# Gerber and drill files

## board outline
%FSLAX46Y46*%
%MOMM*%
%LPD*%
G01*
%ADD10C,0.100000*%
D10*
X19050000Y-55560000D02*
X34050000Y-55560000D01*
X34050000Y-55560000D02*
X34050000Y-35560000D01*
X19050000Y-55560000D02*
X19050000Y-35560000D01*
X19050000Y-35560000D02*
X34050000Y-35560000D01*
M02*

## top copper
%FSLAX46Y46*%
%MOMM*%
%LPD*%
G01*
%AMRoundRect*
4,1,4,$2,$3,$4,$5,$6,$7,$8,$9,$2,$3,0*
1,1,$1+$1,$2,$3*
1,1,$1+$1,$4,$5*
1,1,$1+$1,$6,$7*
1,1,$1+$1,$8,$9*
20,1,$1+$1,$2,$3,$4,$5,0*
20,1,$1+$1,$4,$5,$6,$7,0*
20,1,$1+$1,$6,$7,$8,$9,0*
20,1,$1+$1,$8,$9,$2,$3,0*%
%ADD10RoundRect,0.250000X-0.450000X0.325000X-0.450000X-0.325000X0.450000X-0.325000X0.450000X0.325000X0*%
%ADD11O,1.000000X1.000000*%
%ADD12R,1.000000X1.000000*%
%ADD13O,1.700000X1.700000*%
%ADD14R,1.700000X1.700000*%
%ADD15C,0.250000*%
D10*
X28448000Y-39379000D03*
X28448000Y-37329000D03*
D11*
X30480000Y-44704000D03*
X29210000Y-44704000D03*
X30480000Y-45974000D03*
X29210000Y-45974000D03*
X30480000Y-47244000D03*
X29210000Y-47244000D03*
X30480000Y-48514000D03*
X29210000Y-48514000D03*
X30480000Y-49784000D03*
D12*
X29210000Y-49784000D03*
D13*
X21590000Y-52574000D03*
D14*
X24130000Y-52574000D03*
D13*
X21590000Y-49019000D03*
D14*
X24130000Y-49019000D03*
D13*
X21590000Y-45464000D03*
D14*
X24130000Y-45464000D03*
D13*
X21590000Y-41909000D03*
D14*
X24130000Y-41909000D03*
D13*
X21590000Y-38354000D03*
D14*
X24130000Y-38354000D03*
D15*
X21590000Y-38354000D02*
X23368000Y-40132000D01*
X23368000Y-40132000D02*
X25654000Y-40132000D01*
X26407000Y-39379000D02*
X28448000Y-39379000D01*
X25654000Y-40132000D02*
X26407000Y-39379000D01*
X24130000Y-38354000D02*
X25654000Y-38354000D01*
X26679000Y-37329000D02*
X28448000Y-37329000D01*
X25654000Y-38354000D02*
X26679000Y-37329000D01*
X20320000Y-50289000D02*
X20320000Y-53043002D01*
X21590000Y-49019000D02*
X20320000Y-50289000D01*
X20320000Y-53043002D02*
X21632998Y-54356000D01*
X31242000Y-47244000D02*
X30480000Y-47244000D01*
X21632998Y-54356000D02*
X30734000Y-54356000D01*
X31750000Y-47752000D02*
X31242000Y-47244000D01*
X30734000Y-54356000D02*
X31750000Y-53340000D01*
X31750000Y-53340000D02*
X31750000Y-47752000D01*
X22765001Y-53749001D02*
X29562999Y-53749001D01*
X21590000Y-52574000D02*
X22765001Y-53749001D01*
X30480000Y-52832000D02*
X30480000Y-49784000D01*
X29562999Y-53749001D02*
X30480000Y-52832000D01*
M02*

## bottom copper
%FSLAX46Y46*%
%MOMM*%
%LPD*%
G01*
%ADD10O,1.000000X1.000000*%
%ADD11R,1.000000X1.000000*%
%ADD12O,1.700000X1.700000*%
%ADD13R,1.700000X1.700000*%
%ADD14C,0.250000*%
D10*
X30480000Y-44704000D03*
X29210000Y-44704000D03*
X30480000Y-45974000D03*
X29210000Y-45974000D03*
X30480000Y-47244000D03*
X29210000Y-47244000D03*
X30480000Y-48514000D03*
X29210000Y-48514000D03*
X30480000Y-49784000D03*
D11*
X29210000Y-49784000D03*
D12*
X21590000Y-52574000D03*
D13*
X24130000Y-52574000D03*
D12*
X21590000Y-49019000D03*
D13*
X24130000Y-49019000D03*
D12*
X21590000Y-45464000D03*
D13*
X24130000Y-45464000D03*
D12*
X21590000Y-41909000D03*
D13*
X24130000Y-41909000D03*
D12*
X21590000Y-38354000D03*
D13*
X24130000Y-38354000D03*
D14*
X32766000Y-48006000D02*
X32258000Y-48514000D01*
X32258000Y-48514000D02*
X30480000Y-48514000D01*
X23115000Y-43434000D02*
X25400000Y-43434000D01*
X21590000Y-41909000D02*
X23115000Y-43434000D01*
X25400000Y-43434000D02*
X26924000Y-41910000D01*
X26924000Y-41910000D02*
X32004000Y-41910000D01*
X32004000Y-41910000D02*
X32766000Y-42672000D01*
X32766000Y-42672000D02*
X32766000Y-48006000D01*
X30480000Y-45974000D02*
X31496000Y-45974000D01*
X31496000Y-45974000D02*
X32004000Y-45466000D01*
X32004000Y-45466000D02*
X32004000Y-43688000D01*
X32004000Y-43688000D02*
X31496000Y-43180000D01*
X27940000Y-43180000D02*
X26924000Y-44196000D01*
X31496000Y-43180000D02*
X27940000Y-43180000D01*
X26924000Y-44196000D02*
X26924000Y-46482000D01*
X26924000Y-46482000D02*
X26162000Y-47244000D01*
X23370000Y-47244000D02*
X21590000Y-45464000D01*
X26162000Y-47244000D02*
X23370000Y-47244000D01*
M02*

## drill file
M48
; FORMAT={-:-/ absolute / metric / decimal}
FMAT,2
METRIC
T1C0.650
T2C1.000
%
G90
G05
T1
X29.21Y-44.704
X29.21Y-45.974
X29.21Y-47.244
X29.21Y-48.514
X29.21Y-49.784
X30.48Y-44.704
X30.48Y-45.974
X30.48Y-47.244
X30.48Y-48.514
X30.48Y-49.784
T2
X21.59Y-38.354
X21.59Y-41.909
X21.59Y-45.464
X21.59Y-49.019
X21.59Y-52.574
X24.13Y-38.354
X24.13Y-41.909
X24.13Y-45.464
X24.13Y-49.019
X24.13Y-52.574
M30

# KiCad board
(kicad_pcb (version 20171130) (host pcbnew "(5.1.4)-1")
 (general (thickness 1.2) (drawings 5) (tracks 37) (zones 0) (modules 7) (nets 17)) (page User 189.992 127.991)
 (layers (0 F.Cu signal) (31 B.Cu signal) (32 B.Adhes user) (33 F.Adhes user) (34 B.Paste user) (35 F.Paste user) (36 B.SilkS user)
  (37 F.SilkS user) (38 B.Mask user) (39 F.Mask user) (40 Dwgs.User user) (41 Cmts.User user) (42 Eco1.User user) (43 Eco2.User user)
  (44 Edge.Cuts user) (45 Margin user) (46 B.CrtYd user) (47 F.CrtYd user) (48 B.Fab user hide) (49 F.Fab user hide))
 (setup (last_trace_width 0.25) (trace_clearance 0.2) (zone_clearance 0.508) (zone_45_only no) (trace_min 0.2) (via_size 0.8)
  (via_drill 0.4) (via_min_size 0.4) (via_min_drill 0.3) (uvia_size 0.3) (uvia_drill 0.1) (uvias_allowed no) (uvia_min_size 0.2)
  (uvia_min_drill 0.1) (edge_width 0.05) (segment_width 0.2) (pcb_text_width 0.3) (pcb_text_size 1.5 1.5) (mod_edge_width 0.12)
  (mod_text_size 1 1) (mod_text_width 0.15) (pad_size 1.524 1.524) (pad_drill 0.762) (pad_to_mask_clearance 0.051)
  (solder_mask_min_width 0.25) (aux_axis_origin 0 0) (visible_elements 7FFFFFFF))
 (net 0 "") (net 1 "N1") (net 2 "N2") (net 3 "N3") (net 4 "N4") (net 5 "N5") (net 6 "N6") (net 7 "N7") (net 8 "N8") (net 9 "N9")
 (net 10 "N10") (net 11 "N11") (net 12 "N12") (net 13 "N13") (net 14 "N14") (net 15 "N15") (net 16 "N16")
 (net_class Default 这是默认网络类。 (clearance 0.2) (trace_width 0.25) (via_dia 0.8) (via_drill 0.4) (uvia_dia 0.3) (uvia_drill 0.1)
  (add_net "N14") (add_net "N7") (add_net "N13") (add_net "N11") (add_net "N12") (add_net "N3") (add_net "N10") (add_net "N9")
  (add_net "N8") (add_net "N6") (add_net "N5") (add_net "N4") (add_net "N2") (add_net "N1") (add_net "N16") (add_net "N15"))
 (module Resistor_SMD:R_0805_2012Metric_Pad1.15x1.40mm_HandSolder (layer F.Cu) (at 28.448 38.354 270)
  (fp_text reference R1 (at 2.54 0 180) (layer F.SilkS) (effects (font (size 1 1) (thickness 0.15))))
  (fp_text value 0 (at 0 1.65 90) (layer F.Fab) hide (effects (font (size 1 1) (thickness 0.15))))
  (pad 2 smd roundrect (at 1.025 0 270) (size 1.15 1.4) (layers F.Cu F.Paste F.Mask) (roundrect_rratio 0.217391) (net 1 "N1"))
  (pad 1 smd roundrect (at -1.025 0 270) (size 1.15 1.4) (layers F.Cu F.Paste F.Mask) (roundrect_rratio 0.217391) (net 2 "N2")))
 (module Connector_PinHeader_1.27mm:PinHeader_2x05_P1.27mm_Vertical (layer B.Cu) (at 29.21 49.784)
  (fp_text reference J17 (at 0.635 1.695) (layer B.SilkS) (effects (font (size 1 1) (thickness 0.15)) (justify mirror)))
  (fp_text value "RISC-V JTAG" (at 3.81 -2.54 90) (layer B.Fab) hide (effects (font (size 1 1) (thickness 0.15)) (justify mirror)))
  (pad 10 thru_hole oval (at 1.27 -5.08) (size 1 1) (drill 0.65) (layers *.Cu *.Mask) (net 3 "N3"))
  (pad 9 thru_hole oval (at 0 -5.08) (size 1 1) (drill 0.65) (layers *.Cu *.Mask) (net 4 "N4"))
  (pad 8 thru_hole oval (at 1.27 -3.81) (size 1 1) (drill 0.65) (layers *.Cu *.Mask) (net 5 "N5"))
  (pad 7 thru_hole oval (at 0 -3.81) (size 1 1) (drill 0.65) (layers *.Cu *.Mask) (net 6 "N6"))
  (pad 6 thru_hole oval (at 1.27 -2.54) (size 1 1) (drill 0.65) (layers *.Cu *.Mask) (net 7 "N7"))
  (pad 5 thru_hole oval (at 0 -2.54) (size 1 1) (drill 0.65) (layers *.Cu *.Mask) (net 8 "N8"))
  (pad 4 thru_hole oval (at 1.27 -1.27) (size 1 1) (drill 0.65) (layers *.Cu *.Mask) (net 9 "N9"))
  (pad 3 thru_hole oval (at 0 -1.27) (size 1 1) (drill 0.65) (layers *.Cu *.Mask) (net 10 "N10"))
  (pad 2 thru_hole oval (at 1.27 0) (size 1 1) (drill 0.65) (layers *.Cu *.Mask) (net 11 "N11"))
  (pad 1 thru_hole rect (at 0 0) (size 1 1) (drill 0.65) (layers *.Cu *.Mask) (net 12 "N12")))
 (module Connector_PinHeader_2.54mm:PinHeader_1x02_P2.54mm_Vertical (layer F.Cu) (at 24.13 52.574 270)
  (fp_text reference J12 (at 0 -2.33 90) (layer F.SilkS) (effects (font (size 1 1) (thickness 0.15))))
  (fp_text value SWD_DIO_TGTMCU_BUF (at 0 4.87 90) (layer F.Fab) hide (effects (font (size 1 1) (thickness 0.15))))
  (pad 2 thru_hole oval (at 0 2.54 270) (size 1.7 1.7) (drill 1) (layers *.Cu *.Mask) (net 11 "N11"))
  (pad 1 thru_hole rect (at 0 0 270) (size 1.7 1.7) (drill 1) (layers *.Cu *.Mask) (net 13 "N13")))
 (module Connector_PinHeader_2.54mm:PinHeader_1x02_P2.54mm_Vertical (layer F.Cu) (at 24.13 49.019 270)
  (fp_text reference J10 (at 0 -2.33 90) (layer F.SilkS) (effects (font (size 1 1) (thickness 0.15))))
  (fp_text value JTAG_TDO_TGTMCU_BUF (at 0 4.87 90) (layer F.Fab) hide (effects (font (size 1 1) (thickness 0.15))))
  (pad 2 thru_hole oval (at 0 2.54 270) (size 1.7 1.7) (drill 1) (layers *.Cu *.Mask) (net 7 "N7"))
  (pad 1 thru_hole rect (at 0 0 270) (size 1.7 1.7) (drill 1) (layers *.Cu *.Mask) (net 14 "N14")))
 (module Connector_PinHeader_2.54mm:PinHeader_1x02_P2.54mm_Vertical (layer F.Cu) (at 24.13 45.464 270)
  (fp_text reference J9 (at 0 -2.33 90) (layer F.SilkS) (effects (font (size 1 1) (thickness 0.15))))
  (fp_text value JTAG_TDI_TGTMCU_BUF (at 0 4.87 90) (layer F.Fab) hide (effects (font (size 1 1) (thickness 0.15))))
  (pad 2 thru_hole oval (at 0 2.54 270) (size 1.7 1.7) (drill 1) (layers *.Cu *.Mask) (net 5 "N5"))
  (pad 1 thru_hole rect (at 0 0 270) (size 1.7 1.7) (drill 1) (layers *.Cu *.Mask) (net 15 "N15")))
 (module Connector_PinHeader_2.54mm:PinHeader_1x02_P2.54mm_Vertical (layer F.Cu) (at 24.13 41.909 270)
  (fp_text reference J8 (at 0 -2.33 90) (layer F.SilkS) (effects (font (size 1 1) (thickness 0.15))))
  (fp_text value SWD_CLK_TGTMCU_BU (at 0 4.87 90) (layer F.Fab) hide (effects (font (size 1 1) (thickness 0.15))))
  (pad 2 thru_hole oval (at 0 2.54 270) (size 1.7 1.7) (drill 1) (layers *.Cu *.Mask) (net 9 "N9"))
  (pad 1 thru_hole rect (at 0 0 270) (size 1.7 1.7) (drill 1) (layers *.Cu *.Mask) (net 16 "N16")))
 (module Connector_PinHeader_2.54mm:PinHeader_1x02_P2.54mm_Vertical (layer F.Cu) (at 24.13 38.354 270)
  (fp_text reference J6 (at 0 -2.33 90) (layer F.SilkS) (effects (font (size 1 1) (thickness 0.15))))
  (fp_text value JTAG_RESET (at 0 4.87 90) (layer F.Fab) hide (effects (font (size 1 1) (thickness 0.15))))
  (pad 2 thru_hole oval (at 0 2.54 270) (size 1.7 1.7) (drill 1) (layers *.Cu *.Mask) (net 1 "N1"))
  (pad 1 thru_hole rect (at 0 0 270) (size 1.7 1.7) (drill 1) (layers *.Cu *.Mask) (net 2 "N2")))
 (gr_line (start 19.05 55.56) (end 34.05 55.56) (layer Edge.Cuts) (width 0.1))
 (gr_line (start 34.05 55.56) (end 34.05 35.56) (layer Edge.Cuts) (width 0.1))
 (gr_line (start 19.05 55.56) (end 19.05 35.56) (layer Edge.Cuts) (width 0.1))
 (gr_line (start 19.05 35.56) (end 34.05 35.56) (layer Edge.Cuts) (width 0.1))
 (segment (start 21.59 38.354) (end 23.368 40.132) (width 0.25) (layer F.Cu) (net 1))
 (segment (start 23.368 40.132) (end 25.654 40.132) (width 0.25) (layer F.Cu) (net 1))
 (segment (start 26.407 39.379) (end 28.448 39.379) (width 0.25) (layer F.Cu) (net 1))
 (segment (start 25.654 40.132) (end 26.407 39.379) (width 0.25) (layer F.Cu) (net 1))
 (segment (start 24.13 38.354) (end 25.654 38.354) (width 0.25) (layer F.Cu) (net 2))
 (segment (start 26.679 37.329) (end 28.448 37.329) (width 0.25) (layer F.Cu) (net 2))
 (segment (start 25.654 38.354) (end 26.679 37.329) (width 0.25) (layer F.Cu) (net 2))
 (segment (start 32.766 48.006) (end 32.258 48.514) (width 0.25) (layer B.Cu) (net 9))
 (segment (start 32.258 48.514) (end 30.48 48.514) (width 0.25) (layer B.Cu) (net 9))
 (segment (start 23.115 43.434) (end 25.4 43.434) (width 0.25) (layer B.Cu) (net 9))
 (segment (start 21.59 41.909) (end 23.115 43.434) (width 0.25) (layer B.Cu) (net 9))
 (segment (start 25.4 43.434) (end 26.924 41.91) (width 0.25) (layer B.Cu) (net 9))
 (segment (start 26.924 41.91) (end 32.004 41.91) (width 0.25) (layer B.Cu) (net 9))
 (segment (start 32.004 41.91) (end 32.766 42.672) (width 0.25) (layer B.Cu) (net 9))
 (segment (start 32.766 42.672) (end 32.766 48.006) (width 0.25) (layer B.Cu) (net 9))
 (segment (start 30.48 45.974) (end 31.496 45.974) (width 0.25) (layer B.Cu) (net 5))
 (segment (start 31.496 45.974) (end 32.004 45.466) (width 0.25) (layer B.Cu) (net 5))
 (segment (start 32.004 45.466) (end 32.004 43.688) (width 0.25) (layer B.Cu) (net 5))
 (segment (start 32.004 43.688) (end 31.496 43.18) (width 0.25) (layer B.Cu) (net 5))
 (segment (start 27.94 43.18) (end 26.924 44.196) (width 0.25) (layer B.Cu) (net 5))
 (segment (start 31.496 43.18) (end 27.94 43.18) (width 0.25) (layer B.Cu) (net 5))
 (segment (start 26.924 44.196) (end 26.924 46.482) (width 0.25) (layer B.Cu) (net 5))
 (segment (start 26.924 46.482) (end 26.162 47.244) (width 0.25) (layer B.Cu) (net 5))
 (segment (start 23.37 47.244) (end 21.59 45.464) (width 0.25) (layer B.Cu) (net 5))
 (segment (start 26.162 47.244) (end 23.37 47.244) (width 0.25) (layer B.Cu) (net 5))
 (segment (start 20.32 50.289) (end 20.32 53.043002) (width 0.25) (layer F.Cu) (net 7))
 (segment (start 21.59 49.019) (end 20.32 50.289) (width 0.25) (layer F.Cu) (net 7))
 (segment (start 20.32 53.043002) (end 21.632998 54.356) (width 0.25) (layer F.Cu) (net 7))
 (segment (start 31.242 47.244) (end 30.48 47.244) (width 0.25) (layer F.Cu) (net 7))
 (segment (start 21.632998 54.356) (end 30.734 54.356) (width 0.25) (layer F.Cu) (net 7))
 (segment (start 31.75 47.752) (end 31.242 47.244) (width 0.25) (layer F.Cu) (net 7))
 (segment (start 30.734 54.356) (end 31.75 53.34) (width 0.25) (layer F.Cu) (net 7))
 (segment (start 31.75 53.34) (end 31.75 47.752) (width 0.25) (layer F.Cu) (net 7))
 (segment (start 22.765001 53.749001) (end 29.562999 53.749001) (width 0.25) (layer F.Cu) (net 11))
 (segment (start 21.59 52.574) (end 22.765001 53.749001) (width 0.25) (layer F.Cu) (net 11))
 (segment (start 30.48 52.832) (end 30.48 49.784) (width 0.25) (layer F.Cu) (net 11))
 (segment (start 29.562999 53.749001) (end 30.48 52.832) (width 0.25) (layer F.Cu) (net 11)))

